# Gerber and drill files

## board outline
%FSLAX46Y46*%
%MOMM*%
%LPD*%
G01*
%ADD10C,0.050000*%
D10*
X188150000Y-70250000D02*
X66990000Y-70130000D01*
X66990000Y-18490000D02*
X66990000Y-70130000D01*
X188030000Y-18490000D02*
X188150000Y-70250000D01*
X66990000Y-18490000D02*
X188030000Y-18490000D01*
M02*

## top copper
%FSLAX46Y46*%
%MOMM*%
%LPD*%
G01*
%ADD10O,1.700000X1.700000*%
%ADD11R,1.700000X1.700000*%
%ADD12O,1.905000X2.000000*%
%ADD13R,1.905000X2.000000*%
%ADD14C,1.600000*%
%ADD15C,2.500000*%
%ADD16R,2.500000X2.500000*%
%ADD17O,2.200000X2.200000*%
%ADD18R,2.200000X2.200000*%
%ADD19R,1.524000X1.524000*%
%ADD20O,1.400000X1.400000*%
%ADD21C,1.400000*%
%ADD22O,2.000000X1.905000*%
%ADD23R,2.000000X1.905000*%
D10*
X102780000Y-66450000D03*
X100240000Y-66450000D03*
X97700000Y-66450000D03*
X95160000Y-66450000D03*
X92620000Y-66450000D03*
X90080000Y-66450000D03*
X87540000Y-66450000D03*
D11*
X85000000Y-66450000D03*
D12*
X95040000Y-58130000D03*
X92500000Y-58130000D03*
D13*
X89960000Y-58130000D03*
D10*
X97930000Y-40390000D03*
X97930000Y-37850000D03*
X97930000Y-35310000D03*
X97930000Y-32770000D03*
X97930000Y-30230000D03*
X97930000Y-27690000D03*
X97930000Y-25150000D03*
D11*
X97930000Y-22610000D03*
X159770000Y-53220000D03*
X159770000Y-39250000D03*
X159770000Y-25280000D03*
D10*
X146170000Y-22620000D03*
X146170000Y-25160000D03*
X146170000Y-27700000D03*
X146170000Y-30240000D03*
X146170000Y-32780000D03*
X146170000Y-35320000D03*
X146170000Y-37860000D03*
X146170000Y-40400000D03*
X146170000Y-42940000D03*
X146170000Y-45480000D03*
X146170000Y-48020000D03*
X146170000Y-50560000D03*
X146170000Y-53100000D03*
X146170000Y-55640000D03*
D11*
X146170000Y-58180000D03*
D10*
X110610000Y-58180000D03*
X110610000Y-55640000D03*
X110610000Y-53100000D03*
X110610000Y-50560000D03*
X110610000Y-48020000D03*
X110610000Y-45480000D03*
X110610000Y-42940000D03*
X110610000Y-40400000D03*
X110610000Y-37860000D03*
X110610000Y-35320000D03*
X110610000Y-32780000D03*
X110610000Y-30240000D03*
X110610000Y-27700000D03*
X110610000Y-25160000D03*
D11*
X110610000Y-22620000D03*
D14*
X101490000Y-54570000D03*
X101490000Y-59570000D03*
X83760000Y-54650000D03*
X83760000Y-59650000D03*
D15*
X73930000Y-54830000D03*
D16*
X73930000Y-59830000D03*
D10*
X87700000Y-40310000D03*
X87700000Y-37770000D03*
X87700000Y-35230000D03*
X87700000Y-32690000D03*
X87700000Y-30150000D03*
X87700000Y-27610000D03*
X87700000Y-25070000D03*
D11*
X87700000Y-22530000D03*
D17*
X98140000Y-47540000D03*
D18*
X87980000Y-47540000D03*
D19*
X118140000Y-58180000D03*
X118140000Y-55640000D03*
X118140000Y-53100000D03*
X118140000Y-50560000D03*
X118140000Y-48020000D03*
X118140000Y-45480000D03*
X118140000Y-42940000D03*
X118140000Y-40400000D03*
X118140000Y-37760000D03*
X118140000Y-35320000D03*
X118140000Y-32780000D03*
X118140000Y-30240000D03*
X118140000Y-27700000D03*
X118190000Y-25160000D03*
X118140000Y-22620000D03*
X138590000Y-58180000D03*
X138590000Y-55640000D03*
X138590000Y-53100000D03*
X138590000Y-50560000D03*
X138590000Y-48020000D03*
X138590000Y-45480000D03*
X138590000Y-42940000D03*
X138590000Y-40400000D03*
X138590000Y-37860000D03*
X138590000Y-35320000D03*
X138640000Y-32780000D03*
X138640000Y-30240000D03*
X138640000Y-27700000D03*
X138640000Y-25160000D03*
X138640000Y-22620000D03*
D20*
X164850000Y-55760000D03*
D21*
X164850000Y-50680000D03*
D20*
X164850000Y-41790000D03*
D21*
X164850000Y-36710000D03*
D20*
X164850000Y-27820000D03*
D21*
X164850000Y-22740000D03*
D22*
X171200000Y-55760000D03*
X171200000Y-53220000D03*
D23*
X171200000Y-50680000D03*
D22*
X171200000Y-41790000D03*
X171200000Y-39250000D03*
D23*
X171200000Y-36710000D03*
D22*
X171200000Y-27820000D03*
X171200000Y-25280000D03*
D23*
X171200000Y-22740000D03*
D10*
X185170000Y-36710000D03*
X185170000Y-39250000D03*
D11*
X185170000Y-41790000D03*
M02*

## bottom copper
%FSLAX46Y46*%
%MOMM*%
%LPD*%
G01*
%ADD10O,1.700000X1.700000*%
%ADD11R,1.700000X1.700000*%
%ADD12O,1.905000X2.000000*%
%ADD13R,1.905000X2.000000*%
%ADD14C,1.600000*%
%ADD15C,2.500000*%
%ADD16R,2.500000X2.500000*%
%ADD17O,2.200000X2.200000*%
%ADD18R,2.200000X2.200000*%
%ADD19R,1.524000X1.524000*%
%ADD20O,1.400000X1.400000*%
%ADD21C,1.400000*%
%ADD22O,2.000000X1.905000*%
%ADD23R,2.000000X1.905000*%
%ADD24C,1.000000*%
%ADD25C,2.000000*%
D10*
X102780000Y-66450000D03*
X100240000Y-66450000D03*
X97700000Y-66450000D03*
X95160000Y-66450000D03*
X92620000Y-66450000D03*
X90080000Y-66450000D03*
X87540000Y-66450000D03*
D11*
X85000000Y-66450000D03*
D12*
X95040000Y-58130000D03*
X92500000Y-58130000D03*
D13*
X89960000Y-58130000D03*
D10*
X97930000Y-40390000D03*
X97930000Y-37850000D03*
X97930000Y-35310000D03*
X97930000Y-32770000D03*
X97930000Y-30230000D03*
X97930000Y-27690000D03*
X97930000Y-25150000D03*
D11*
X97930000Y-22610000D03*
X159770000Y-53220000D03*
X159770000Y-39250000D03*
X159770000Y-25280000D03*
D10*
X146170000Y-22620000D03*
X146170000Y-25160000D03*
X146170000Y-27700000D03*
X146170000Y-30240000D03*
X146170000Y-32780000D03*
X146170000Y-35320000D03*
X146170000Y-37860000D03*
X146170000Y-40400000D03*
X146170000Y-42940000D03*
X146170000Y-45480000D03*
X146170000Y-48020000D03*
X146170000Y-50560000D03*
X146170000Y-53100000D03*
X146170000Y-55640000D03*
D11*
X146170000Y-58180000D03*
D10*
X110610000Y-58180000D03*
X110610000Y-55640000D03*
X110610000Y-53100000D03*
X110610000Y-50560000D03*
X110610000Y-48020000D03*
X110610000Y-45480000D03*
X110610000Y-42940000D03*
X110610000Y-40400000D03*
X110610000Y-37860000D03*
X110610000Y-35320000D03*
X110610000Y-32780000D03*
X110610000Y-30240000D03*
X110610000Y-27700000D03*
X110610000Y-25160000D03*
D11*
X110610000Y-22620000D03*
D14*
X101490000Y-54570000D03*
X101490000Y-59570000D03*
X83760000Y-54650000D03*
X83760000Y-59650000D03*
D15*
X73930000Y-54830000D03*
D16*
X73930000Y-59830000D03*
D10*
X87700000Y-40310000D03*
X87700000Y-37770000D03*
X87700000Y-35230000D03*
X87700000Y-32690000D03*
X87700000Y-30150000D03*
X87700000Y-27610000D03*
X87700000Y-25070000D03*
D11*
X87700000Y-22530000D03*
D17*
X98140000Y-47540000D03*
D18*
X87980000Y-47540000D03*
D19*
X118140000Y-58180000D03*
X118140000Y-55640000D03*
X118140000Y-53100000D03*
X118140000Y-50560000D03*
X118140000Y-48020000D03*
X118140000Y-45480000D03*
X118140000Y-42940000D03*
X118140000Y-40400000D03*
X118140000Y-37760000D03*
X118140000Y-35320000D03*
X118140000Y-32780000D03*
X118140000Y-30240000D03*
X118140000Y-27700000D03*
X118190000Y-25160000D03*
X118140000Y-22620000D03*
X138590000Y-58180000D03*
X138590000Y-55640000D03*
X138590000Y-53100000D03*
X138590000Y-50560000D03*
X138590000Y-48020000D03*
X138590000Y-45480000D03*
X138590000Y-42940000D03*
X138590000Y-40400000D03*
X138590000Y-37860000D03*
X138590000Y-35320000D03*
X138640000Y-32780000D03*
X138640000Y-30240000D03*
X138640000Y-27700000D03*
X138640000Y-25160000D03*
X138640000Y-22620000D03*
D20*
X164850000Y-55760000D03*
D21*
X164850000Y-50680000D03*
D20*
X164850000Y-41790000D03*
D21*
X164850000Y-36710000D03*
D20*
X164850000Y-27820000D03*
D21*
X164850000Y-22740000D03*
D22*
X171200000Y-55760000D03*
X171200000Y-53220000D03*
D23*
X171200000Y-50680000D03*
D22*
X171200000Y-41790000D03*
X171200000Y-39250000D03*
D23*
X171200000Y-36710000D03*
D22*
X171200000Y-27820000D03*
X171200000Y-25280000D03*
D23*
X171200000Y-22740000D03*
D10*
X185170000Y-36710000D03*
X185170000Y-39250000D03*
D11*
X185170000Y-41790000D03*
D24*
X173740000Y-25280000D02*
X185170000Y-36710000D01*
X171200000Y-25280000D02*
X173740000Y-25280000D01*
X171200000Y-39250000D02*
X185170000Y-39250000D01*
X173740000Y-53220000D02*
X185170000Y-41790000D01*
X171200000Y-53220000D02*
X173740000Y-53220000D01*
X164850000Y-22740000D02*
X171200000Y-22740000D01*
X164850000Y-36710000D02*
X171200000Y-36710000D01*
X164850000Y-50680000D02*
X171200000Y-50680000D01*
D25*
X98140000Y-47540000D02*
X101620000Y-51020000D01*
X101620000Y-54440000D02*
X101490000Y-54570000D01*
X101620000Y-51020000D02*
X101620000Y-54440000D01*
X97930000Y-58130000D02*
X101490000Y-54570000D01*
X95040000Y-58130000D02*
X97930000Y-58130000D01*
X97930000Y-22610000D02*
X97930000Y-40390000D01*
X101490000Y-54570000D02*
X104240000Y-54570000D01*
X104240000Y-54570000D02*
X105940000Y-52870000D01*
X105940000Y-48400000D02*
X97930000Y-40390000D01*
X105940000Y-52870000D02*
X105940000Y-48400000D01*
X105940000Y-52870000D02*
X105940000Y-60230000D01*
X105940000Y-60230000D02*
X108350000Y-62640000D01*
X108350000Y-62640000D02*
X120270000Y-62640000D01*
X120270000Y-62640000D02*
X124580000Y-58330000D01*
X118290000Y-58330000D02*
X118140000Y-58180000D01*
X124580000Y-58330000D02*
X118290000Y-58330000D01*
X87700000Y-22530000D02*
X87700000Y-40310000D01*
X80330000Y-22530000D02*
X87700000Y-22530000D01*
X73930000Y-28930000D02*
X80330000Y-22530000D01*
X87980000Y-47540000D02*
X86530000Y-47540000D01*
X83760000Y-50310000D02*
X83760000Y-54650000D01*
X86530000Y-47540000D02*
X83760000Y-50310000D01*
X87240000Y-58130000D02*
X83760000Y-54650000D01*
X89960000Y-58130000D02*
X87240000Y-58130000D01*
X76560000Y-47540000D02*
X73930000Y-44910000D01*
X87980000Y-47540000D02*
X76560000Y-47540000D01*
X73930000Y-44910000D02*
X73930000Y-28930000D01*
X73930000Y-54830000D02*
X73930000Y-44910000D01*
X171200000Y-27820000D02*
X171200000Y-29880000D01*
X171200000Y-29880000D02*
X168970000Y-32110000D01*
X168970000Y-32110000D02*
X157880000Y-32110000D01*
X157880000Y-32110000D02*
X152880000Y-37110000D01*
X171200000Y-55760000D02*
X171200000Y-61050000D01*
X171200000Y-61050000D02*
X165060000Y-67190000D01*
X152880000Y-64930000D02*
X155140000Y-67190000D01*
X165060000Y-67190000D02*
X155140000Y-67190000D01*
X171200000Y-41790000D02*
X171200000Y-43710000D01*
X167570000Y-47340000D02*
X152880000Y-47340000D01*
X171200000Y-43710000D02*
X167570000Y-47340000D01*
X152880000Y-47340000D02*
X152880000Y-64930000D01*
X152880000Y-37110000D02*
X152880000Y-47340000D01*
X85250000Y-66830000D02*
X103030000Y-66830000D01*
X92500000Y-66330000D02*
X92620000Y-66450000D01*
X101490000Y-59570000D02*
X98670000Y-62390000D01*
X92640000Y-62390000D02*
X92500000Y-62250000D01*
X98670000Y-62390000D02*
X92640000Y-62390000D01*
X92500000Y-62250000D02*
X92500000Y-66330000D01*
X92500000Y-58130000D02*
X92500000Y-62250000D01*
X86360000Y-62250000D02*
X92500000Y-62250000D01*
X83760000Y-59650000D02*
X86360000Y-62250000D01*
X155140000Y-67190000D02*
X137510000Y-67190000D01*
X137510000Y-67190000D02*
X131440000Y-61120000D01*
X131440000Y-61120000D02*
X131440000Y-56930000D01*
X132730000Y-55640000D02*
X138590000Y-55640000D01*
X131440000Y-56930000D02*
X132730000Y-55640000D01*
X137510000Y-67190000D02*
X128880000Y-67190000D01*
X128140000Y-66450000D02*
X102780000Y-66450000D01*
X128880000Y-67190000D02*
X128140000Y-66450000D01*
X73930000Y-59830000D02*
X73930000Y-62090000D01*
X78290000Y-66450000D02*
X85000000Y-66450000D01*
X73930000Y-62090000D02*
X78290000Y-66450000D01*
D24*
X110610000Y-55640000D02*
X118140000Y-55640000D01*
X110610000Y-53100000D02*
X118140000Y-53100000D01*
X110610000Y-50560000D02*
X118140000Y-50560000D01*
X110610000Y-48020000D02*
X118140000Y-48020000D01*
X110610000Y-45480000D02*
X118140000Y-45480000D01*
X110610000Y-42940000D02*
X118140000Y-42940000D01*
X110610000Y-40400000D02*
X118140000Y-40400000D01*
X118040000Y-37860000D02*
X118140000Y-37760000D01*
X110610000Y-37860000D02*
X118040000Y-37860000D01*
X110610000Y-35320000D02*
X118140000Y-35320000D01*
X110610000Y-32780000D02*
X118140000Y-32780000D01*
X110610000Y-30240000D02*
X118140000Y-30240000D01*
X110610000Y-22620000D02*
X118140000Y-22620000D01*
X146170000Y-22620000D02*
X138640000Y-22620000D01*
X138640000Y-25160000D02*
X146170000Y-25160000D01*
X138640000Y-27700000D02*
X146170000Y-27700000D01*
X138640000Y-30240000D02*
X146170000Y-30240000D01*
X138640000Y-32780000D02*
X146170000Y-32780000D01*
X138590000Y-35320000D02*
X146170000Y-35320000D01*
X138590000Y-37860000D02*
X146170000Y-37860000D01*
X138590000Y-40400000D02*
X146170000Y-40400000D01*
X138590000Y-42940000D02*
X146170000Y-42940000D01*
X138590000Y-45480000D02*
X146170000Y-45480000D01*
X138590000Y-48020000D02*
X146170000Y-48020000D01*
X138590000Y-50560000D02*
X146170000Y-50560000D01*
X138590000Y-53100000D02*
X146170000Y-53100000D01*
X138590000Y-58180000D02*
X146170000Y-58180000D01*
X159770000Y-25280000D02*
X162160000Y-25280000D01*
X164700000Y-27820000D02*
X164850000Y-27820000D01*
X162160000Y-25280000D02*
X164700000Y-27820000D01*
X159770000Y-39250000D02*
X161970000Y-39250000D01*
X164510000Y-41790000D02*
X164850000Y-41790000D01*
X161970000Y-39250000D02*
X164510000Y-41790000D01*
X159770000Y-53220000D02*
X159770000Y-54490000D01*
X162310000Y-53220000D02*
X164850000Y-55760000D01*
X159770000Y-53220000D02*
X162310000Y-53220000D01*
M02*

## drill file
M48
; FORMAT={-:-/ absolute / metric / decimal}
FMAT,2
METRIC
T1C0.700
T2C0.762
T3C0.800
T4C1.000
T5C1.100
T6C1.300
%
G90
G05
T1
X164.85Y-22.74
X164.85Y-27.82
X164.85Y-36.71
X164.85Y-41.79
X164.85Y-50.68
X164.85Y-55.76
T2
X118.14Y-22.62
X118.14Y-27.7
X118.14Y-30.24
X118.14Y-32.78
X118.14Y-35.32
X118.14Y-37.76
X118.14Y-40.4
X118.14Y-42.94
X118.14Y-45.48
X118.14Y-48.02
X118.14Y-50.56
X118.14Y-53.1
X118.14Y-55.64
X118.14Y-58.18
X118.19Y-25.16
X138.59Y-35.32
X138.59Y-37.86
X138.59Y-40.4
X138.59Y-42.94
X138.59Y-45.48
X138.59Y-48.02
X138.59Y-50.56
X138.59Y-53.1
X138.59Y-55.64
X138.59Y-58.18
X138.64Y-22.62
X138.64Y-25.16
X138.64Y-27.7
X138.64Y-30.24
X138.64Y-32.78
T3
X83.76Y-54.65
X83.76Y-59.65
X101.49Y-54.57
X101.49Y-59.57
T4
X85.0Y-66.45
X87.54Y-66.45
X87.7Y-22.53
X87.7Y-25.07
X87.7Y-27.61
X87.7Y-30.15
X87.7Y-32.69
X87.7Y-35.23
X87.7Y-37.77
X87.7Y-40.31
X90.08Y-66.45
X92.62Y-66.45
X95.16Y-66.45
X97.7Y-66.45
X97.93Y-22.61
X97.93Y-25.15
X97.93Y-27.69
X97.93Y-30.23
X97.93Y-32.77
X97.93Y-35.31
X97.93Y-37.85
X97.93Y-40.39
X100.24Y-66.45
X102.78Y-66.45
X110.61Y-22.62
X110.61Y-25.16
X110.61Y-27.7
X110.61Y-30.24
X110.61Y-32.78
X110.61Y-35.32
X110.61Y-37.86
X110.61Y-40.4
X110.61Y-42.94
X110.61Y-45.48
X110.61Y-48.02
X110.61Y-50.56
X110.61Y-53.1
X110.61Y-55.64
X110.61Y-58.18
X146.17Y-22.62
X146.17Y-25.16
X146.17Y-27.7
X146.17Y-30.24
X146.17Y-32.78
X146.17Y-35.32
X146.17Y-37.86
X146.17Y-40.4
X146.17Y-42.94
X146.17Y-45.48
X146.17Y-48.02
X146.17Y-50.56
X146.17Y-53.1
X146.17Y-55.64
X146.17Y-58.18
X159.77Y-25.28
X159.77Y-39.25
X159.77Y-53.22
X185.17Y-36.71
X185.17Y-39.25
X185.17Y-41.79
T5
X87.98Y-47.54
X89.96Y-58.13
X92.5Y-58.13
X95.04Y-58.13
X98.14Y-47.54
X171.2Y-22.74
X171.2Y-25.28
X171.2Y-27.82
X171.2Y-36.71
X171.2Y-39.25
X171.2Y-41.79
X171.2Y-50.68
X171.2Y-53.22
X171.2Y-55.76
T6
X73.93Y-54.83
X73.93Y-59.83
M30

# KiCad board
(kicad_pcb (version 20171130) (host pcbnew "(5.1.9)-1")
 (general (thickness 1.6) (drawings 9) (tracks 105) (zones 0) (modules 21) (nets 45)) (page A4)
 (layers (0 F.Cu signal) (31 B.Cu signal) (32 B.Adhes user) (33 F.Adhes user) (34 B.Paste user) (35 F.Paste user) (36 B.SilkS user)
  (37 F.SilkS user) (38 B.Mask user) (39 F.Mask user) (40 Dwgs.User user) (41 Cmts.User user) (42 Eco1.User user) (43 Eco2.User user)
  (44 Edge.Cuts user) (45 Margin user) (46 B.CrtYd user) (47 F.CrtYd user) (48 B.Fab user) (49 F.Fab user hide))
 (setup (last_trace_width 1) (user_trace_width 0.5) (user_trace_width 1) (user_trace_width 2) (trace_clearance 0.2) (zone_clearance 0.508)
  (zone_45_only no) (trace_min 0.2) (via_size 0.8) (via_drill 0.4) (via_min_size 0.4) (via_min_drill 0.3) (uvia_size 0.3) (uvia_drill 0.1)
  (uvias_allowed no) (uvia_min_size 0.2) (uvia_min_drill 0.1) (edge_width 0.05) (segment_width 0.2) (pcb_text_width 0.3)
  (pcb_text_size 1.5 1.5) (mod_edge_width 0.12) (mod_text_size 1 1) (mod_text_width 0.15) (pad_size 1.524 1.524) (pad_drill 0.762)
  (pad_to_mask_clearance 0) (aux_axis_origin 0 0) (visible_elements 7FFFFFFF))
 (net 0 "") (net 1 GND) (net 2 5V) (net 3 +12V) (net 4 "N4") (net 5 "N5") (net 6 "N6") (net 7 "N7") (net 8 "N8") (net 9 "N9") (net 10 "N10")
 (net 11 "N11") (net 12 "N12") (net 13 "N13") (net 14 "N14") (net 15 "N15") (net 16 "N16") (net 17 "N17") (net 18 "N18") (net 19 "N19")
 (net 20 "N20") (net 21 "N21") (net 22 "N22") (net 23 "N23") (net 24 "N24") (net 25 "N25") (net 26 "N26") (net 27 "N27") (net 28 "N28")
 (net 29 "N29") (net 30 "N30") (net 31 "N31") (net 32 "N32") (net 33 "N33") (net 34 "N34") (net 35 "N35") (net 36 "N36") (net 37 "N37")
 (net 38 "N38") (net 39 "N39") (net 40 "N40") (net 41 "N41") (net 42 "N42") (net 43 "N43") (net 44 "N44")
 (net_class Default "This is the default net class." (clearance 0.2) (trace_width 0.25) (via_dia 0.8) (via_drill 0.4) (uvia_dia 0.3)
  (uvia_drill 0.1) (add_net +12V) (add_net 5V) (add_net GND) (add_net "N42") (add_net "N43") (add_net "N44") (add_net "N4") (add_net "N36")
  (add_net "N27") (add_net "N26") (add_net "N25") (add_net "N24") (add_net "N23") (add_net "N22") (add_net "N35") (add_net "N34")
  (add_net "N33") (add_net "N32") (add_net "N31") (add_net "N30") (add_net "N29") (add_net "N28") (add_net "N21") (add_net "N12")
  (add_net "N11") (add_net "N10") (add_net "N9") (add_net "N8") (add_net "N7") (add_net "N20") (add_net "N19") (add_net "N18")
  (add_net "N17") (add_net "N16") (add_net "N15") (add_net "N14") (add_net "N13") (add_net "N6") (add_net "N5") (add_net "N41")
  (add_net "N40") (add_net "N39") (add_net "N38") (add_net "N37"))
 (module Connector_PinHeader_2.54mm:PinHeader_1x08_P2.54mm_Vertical (layer F.Cu) (at 85 66.45 90)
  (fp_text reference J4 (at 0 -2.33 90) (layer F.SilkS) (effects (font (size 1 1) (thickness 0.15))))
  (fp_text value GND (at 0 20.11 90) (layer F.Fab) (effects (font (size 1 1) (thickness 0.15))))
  (pad 8 thru_hole oval (at 0 17.78 90) (size 1.7 1.7) (drill 1) (layers *.Cu *.Mask) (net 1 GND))
  (pad 7 thru_hole oval (at 0 15.24 90) (size 1.7 1.7) (drill 1) (layers *.Cu *.Mask) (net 1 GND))
  (pad 6 thru_hole oval (at 0 12.7 90) (size 1.7 1.7) (drill 1) (layers *.Cu *.Mask) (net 1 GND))
  (pad 5 thru_hole oval (at 0 10.16 90) (size 1.7 1.7) (drill 1) (layers *.Cu *.Mask) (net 1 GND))
  (pad 4 thru_hole oval (at 0 7.62 90) (size 1.7 1.7) (drill 1) (layers *.Cu *.Mask) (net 1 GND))
  (pad 3 thru_hole oval (at 0 5.08 90) (size 1.7 1.7) (drill 1) (layers *.Cu *.Mask) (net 1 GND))
  (pad 2 thru_hole oval (at 0 2.54 90) (size 1.7 1.7) (drill 1) (layers *.Cu *.Mask) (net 1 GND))
  (pad 1 thru_hole rect (at 0 0 90) (size 1.7 1.7) (drill 1) (layers *.Cu *.Mask) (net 1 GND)))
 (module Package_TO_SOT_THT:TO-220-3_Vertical (layer F.Cu) (at 89.96 58.13)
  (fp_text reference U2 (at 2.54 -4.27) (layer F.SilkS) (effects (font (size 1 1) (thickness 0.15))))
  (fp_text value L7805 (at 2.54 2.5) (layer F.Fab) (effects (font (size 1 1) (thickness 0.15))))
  (pad 3 thru_hole oval (at 5.08 0) (size 1.905 2) (drill 1.1) (layers *.Cu *.Mask) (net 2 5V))
  (pad 2 thru_hole oval (at 2.54 0) (size 1.905 2) (drill 1.1) (layers *.Cu *.Mask) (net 1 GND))
  (pad 1 thru_hole rect (at 0 0) (size 1.905 2) (drill 1.1) (layers *.Cu *.Mask) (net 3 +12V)))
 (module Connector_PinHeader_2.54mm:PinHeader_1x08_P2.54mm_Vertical (layer F.Cu) (at 97.93 22.61)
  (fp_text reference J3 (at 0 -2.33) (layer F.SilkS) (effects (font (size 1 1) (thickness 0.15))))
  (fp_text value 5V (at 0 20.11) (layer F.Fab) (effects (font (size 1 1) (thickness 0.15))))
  (pad 8 thru_hole oval (at 0 17.78) (size 1.7 1.7) (drill 1) (layers *.Cu *.Mask) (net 2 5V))
  (pad 7 thru_hole oval (at 0 15.24) (size 1.7 1.7) (drill 1) (layers *.Cu *.Mask) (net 2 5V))
  (pad 6 thru_hole oval (at 0 12.7) (size 1.7 1.7) (drill 1) (layers *.Cu *.Mask) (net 2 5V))
  (pad 5 thru_hole oval (at 0 10.16) (size 1.7 1.7) (drill 1) (layers *.Cu *.Mask) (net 2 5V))
  (pad 4 thru_hole oval (at 0 7.62) (size 1.7 1.7) (drill 1) (layers *.Cu *.Mask) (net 2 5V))
  (pad 3 thru_hole oval (at 0 5.08) (size 1.7 1.7) (drill 1) (layers *.Cu *.Mask) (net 2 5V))
  (pad 2 thru_hole oval (at 0 2.54) (size 1.7 1.7) (drill 1) (layers *.Cu *.Mask) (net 2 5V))
  (pad 1 thru_hole rect (at 0 0) (size 1.7 1.7) (drill 1) (layers *.Cu *.Mask) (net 2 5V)))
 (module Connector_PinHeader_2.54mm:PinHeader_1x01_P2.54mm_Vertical (layer F.Cu) (at 159.77 53.22)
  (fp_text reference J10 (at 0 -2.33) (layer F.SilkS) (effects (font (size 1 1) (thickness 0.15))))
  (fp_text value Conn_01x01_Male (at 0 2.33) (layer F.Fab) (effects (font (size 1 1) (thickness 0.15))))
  (pad 1 thru_hole rect (at 0 0) (size 1.7 1.7) (drill 1) (layers *.Cu *.Mask) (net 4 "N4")))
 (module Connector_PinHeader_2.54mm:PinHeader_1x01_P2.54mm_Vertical (layer F.Cu) (at 159.77 39.25)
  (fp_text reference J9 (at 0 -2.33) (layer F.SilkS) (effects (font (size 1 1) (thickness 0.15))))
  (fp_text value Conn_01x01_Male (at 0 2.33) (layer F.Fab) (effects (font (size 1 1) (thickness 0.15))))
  (pad 1 thru_hole rect (at 0 0) (size 1.7 1.7) (drill 1) (layers *.Cu *.Mask) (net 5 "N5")))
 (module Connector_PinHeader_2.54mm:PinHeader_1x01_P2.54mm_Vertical (layer F.Cu) (at 159.77 25.28)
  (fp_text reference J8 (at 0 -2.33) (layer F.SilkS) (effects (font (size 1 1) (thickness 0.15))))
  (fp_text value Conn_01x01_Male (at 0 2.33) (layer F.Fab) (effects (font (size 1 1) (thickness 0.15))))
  (pad 1 thru_hole rect (at 0 0) (size 1.7 1.7) (drill 1) (layers *.Cu *.Mask) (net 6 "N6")))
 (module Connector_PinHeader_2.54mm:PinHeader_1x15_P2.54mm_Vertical (layer F.Cu) (at 146.17 58.18 180)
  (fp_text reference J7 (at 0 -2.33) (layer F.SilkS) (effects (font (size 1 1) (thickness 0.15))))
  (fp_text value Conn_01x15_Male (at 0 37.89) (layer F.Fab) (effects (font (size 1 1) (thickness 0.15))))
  (pad 15 thru_hole oval (at 0 35.56 180) (size 1.7 1.7) (drill 1) (layers *.Cu *.Mask) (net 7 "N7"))
  (pad 14 thru_hole oval (at 0 33.02 180) (size 1.7 1.7) (drill 1) (layers *.Cu *.Mask) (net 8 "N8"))
  (pad 13 thru_hole oval (at 0 30.48 180) (size 1.7 1.7) (drill 1) (layers *.Cu *.Mask) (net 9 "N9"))
  (pad 12 thru_hole oval (at 0 27.94 180) (size 1.7 1.7) (drill 1) (layers *.Cu *.Mask) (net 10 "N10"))
  (pad 11 thru_hole oval (at 0 25.4 180) (size 1.7 1.7) (drill 1) (layers *.Cu *.Mask) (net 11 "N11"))
  (pad 10 thru_hole oval (at 0 22.86 180) (size 1.7 1.7) (drill 1) (layers *.Cu *.Mask) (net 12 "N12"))
  (pad 9 thru_hole oval (at 0 20.32 180) (size 1.7 1.7) (drill 1) (layers *.Cu *.Mask) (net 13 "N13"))
  (pad 8 thru_hole oval (at 0 17.78 180) (size 1.7 1.7) (drill 1) (layers *.Cu *.Mask) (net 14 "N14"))
  (pad 7 thru_hole oval (at 0 15.24 180) (size 1.7 1.7) (drill 1) (layers *.Cu *.Mask) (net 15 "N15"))
  (pad 6 thru_hole oval (at 0 12.7 180) (size 1.7 1.7) (drill 1) (layers *.Cu *.Mask) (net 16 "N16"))
  (pad 5 thru_hole oval (at 0 10.16 180) (size 1.7 1.7) (drill 1) (layers *.Cu *.Mask) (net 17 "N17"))
  (pad 4 thru_hole oval (at 0 7.62 180) (size 1.7 1.7) (drill 1) (layers *.Cu *.Mask) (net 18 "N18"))
  (pad 3 thru_hole oval (at 0 5.08 180) (size 1.7 1.7) (drill 1) (layers *.Cu *.Mask) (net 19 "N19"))
  (pad 2 thru_hole oval (at 0 2.54 180) (size 1.7 1.7) (drill 1) (layers *.Cu *.Mask) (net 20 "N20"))
  (pad 1 thru_hole rect (at 0 0 180) (size 1.7 1.7) (drill 1) (layers *.Cu *.Mask) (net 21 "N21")))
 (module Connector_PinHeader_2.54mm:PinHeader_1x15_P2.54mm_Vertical (layer F.Cu) (at 110.61 22.62)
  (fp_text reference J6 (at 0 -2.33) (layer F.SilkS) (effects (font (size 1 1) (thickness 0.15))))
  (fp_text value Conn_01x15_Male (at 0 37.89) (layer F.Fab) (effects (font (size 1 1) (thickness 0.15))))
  (pad 15 thru_hole oval (at 0 35.56) (size 1.7 1.7) (drill 1) (layers *.Cu *.Mask) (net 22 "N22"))
  (pad 14 thru_hole oval (at 0 33.02) (size 1.7 1.7) (drill 1) (layers *.Cu *.Mask) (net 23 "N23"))
  (pad 13 thru_hole oval (at 0 30.48) (size 1.7 1.7) (drill 1) (layers *.Cu *.Mask) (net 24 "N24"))
  (pad 12 thru_hole oval (at 0 27.94) (size 1.7 1.7) (drill 1) (layers *.Cu *.Mask) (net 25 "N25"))
  (pad 11 thru_hole oval (at 0 25.4) (size 1.7 1.7) (drill 1) (layers *.Cu *.Mask) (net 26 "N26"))
  (pad 10 thru_hole oval (at 0 22.86) (size 1.7 1.7) (drill 1) (layers *.Cu *.Mask) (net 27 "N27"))
  (pad 9 thru_hole oval (at 0 20.32) (size 1.7 1.7) (drill 1) (layers *.Cu *.Mask) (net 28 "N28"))
  (pad 8 thru_hole oval (at 0 17.78) (size 1.7 1.7) (drill 1) (layers *.Cu *.Mask) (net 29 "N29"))
  (pad 7 thru_hole oval (at 0 15.24) (size 1.7 1.7) (drill 1) (layers *.Cu *.Mask) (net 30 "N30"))
  (pad 6 thru_hole oval (at 0 12.7) (size 1.7 1.7) (drill 1) (layers *.Cu *.Mask) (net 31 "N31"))
  (pad 5 thru_hole oval (at 0 10.16) (size 1.7 1.7) (drill 1) (layers *.Cu *.Mask) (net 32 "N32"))
  (pad 4 thru_hole oval (at 0 7.62) (size 1.7 1.7) (drill 1) (layers *.Cu *.Mask) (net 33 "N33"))
  (pad 3 thru_hole oval (at 0 5.08) (size 1.7 1.7) (drill 1) (layers *.Cu *.Mask) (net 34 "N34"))
  (pad 2 thru_hole oval (at 0 2.54) (size 1.7 1.7) (drill 1) (layers *.Cu *.Mask) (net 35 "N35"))
  (pad 1 thru_hole rect (at 0 0) (size 1.7 1.7) (drill 1) (layers *.Cu *.Mask) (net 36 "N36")))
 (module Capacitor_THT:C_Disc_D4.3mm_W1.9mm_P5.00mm (layer F.Cu) (at 101.49 59.57 90)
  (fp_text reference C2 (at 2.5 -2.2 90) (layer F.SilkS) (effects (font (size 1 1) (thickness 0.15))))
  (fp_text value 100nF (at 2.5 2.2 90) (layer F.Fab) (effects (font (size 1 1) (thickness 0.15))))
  (pad 2 thru_hole circle (at 5 0 90) (size 1.6 1.6) (drill 0.8) (layers *.Cu *.Mask) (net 2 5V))
  (pad 1 thru_hole circle (at 0 0 90) (size 1.6 1.6) (drill 0.8) (layers *.Cu *.Mask) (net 1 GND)))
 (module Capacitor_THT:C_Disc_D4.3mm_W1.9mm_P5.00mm (layer F.Cu) (at 83.76 59.65 90)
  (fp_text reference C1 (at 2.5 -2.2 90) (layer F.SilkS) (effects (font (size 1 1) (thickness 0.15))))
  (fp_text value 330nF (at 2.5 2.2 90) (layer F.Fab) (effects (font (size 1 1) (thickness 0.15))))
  (pad 2 thru_hole circle (at 5 0 90) (size 1.6 1.6) (drill 0.8) (layers *.Cu *.Mask) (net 3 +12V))
  (pad 1 thru_hole circle (at 0 0 90) (size 1.6 1.6) (drill 0.8) (layers *.Cu *.Mask) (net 1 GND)))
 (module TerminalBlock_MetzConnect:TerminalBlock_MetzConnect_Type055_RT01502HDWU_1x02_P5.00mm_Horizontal (layer F.Cu) (at 73.93 59.83 90)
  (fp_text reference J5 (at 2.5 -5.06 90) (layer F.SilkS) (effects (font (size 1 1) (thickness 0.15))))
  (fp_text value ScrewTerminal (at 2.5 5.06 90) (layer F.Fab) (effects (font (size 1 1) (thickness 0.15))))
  (pad 2 thru_hole circle (at 5 0 90) (size 2.5 2.5) (drill 1.3) (layers *.Cu *.Mask) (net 3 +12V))
  (pad 1 thru_hole rect (at 0 0 90) (size 2.5 2.5) (drill 1.3) (layers *.Cu *.Mask) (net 1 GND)))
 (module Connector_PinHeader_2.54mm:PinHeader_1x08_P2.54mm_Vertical (layer F.Cu) (at 87.7 22.53)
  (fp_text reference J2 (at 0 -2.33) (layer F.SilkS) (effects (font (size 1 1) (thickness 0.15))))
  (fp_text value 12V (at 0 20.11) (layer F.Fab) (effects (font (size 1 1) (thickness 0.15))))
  (pad 8 thru_hole oval (at 0 17.78) (size 1.7 1.7) (drill 1) (layers *.Cu *.Mask) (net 3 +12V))
  (pad 7 thru_hole oval (at 0 15.24) (size 1.7 1.7) (drill 1) (layers *.Cu *.Mask) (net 3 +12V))
  (pad 6 thru_hole oval (at 0 12.7) (size 1.7 1.7) (drill 1) (layers *.Cu *.Mask) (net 3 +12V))
  (pad 5 thru_hole oval (at 0 10.16) (size 1.7 1.7) (drill 1) (layers *.Cu *.Mask) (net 3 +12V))
  (pad 4 thru_hole oval (at 0 7.62) (size 1.7 1.7) (drill 1) (layers *.Cu *.Mask) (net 3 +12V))
  (pad 3 thru_hole oval (at 0 5.08) (size 1.7 1.7) (drill 1) (layers *.Cu *.Mask) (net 3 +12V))
  (pad 2 thru_hole oval (at 0 2.54) (size 1.7 1.7) (drill 1) (layers *.Cu *.Mask) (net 3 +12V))
  (pad 1 thru_hole rect (at 0 0) (size 1.7 1.7) (drill 1) (layers *.Cu *.Mask) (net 3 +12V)))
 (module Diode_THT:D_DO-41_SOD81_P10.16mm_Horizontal (layer F.Cu) (at 87.98 47.54)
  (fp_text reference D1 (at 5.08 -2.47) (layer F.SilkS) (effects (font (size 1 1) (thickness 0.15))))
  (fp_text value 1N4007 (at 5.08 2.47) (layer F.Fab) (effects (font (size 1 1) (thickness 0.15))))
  (pad 2 thru_hole oval (at 10.16 0) (size 2.2 2.2) (drill 1.1) (layers *.Cu *.Mask) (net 2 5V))
  (pad 1 thru_hole rect (at 0 0) (size 2.2 2.2) (drill 1.1) (layers *.Cu *.Mask) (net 3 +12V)))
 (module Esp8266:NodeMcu (layer F.Cu) (at 128.39 37.86)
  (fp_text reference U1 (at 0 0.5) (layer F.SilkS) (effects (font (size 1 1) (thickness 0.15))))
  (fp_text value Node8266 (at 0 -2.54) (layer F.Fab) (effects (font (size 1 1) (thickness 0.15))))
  (pad 30 thru_hole rect (at -10.25 20.32) (size 1.524 1.524) (drill 0.762) (layers *.Cu *.Mask) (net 2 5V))
  (pad 29 thru_hole rect (at -10.25 17.78) (size 1.524 1.524) (drill 0.762) (layers *.Cu *.Mask) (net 23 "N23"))
  (pad 28 thru_hole rect (at -10.25 15.24) (size 1.524 1.524) (drill 0.762) (layers *.Cu *.Mask) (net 24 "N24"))
  (pad 27 thru_hole rect (at -10.25 12.7) (size 1.524 1.524) (drill 0.762) (layers *.Cu *.Mask) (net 25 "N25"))
  (pad 26 thru_hole rect (at -10.25 10.16) (size 1.524 1.524) (drill 0.762) (layers *.Cu *.Mask) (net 26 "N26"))
  (pad 25 thru_hole rect (at -10.25 7.62) (size 1.524 1.524) (drill 0.762) (layers *.Cu *.Mask) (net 27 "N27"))
  (pad 24 thru_hole rect (at -10.25 5.08) (size 1.524 1.524) (drill 0.762) (layers *.Cu *.Mask) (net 28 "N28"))
  (pad 23 thru_hole rect (at -10.25 2.54) (size 1.524 1.524) (drill 0.762) (layers *.Cu *.Mask) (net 29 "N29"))
  (pad 22 thru_hole rect (at -10.25 -0.1) (size 1.524 1.524) (drill 0.762) (layers *.Cu *.Mask) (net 30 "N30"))
  (pad 21 thru_hole rect (at -10.25 -2.54) (size 1.524 1.524) (drill 0.762) (layers *.Cu *.Mask) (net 31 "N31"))
  (pad 20 thru_hole rect (at -10.25 -5.08) (size 1.524 1.524) (drill 0.762) (layers *.Cu *.Mask) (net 32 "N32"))
  (pad 19 thru_hole rect (at -10.25 -7.62) (size 1.524 1.524) (drill 0.762) (layers *.Cu *.Mask) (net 33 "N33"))
  (pad 18 thru_hole rect (at -10.25 -10.16) (size 1.524 1.524) (drill 0.762) (layers *.Cu *.Mask) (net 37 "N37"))
  (pad 17 thru_hole rect (at -10.2 -12.7) (size 1.524 1.524) (drill 0.762) (layers *.Cu *.Mask) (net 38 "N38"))
  (pad 16 thru_hole rect (at -10.25 -15.24) (size 1.524 1.524) (drill 0.762) (layers *.Cu *.Mask) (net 36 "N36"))
  (pad 15 thru_hole rect (at 10.2 20.32) (size 1.524 1.524) (drill 0.762) (layers *.Cu *.Mask) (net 21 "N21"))
  (pad 14 thru_hole rect (at 10.2 17.78) (size 1.524 1.524) (drill 0.762) (layers *.Cu *.Mask) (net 1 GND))
  (pad 13 thru_hole rect (at 10.2 15.24) (size 1.524 1.524) (drill 0.762) (layers *.Cu *.Mask) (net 19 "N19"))
  (pad 12 thru_hole rect (at 10.2 12.7) (size 1.524 1.524) (drill 0.762) (layers *.Cu *.Mask) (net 18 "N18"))
  (pad 11 thru_hole rect (at 10.2 10.16) (size 1.524 1.524) (drill 0.762) (layers *.Cu *.Mask) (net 17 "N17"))
  (pad 10 thru_hole rect (at 10.2 7.62) (size 1.524 1.524) (drill 0.762) (layers *.Cu *.Mask) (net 16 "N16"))
  (pad 9 thru_hole rect (at 10.2 5.08 90) (size 1.524 1.524) (drill 0.762) (layers *.Cu *.Mask) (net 15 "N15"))
  (pad 8 thru_hole rect (at 10.2 2.54) (size 1.524 1.524) (drill 0.762) (layers *.Cu *.Mask) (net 14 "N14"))
  (pad 7 thru_hole rect (at 10.2 0) (size 1.524 1.524) (drill 0.762) (layers *.Cu *.Mask) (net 13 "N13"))
  (pad 6 thru_hole rect (at 10.2 -2.54) (size 1.524 1.524) (drill 0.762) (layers *.Cu *.Mask) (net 12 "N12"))
  (pad 5 thru_hole rect (at 10.25 -5.08) (size 1.524 1.524) (drill 0.762) (layers *.Cu *.Mask) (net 11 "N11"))
  (pad 4 thru_hole rect (at 10.25 -7.62) (size 1.524 1.524) (drill 0.762) (layers *.Cu *.Mask) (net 10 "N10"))
  (pad 3 thru_hole rect (at 10.25 -10.16) (size 1.524 1.524) (drill 0.762) (layers *.Cu *.Mask) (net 9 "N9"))
  (pad 2 thru_hole rect (at 10.25 -12.7) (size 1.524 1.524) (drill 0.762) (layers *.Cu *.Mask) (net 8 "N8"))
  (pad 1 thru_hole rect (at 10.25 -15.24) (size 1.524 1.524) (drill 0.762) (layers *.Cu *.Mask) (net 7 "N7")))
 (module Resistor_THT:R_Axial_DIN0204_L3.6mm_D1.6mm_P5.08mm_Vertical (layer F.Cu) (at 164.85 50.68 270)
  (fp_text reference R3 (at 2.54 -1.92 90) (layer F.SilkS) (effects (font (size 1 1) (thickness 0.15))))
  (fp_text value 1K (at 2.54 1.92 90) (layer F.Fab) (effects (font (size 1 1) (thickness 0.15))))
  (pad 2 thru_hole oval (at 5.08 0 270) (size 1.4 1.4) (drill 0.7) (layers *.Cu *.Mask) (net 4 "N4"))
  (pad 1 thru_hole circle (at 0 0 270) (size 1.4 1.4) (drill 0.7) (layers *.Cu *.Mask) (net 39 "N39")))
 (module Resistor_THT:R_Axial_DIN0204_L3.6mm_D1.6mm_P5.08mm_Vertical (layer F.Cu) (at 164.85 36.71 270)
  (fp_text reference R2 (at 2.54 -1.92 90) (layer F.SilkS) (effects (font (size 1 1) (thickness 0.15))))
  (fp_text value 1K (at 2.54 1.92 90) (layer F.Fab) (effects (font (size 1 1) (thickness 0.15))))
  (pad 2 thru_hole oval (at 5.08 0 270) (size 1.4 1.4) (drill 0.7) (layers *.Cu *.Mask) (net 5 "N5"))
  (pad 1 thru_hole circle (at 0 0 270) (size 1.4 1.4) (drill 0.7) (layers *.Cu *.Mask) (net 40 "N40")))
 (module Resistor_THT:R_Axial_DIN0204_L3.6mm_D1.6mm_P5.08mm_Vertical (layer F.Cu) (at 164.85 22.74 270)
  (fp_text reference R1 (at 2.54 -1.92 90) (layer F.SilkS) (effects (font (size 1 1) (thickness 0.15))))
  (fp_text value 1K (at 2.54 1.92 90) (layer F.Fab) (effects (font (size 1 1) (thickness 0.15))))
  (pad 2 thru_hole oval (at 5.08 0 270) (size 1.4 1.4) (drill 0.7) (layers *.Cu *.Mask) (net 6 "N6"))
  (pad 1 thru_hole circle (at 0 0 270) (size 1.4 1.4) (drill 0.7) (layers *.Cu *.Mask) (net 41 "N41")))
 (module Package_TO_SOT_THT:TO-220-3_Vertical (layer F.Cu) (at 171.2 50.68 270)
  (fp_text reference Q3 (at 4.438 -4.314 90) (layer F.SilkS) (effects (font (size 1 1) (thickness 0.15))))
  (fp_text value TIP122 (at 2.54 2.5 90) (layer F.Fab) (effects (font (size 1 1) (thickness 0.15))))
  (pad 3 thru_hole oval (at 5.08 0 270) (size 1.905 2) (drill 1.1) (layers *.Cu *.Mask) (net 1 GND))
  (pad 2 thru_hole oval (at 2.54 0 270) (size 1.905 2) (drill 1.1) (layers *.Cu *.Mask) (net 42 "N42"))
  (pad 1 thru_hole rect (at 0 0 270) (size 1.905 2) (drill 1.1) (layers *.Cu *.Mask) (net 39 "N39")))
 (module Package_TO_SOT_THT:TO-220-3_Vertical (layer F.Cu) (at 171.2 36.71 270)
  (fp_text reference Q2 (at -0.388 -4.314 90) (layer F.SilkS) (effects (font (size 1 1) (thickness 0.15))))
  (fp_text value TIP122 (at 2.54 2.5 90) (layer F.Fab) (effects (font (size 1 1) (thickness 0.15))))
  (pad 3 thru_hole oval (at 5.08 0 270) (size 1.905 2) (drill 1.1) (layers *.Cu *.Mask) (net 1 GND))
  (pad 2 thru_hole oval (at 2.54 0 270) (size 1.905 2) (drill 1.1) (layers *.Cu *.Mask) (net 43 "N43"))
  (pad 1 thru_hole rect (at 0 0 270) (size 1.905 2) (drill 1.1) (layers *.Cu *.Mask) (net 40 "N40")))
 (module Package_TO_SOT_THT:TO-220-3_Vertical (layer F.Cu) (at 171.2 22.74 270)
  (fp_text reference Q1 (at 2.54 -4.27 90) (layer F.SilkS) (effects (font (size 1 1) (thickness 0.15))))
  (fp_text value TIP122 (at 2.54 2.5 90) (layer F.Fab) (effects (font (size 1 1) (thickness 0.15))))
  (pad 3 thru_hole oval (at 5.08 0 270) (size 1.905 2) (drill 1.1) (layers *.Cu *.Mask) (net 1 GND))
  (pad 2 thru_hole oval (at 2.54 0 270) (size 1.905 2) (drill 1.1) (layers *.Cu *.Mask) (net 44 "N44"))
  (pad 1 thru_hole rect (at 0 0 270) (size 1.905 2) (drill 1.1) (layers *.Cu *.Mask) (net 41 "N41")))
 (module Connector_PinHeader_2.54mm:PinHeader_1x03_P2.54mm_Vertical (layer F.Cu) (at 185.17 41.79 180)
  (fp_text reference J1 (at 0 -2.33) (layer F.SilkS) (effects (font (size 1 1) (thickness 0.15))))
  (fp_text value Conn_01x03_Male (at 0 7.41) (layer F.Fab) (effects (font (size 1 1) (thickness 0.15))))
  (pad 3 thru_hole oval (at 0 5.08 180) (size 1.7 1.7) (drill 1) (layers *.Cu *.Mask) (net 44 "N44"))
  (pad 2 thru_hole oval (at 0 2.54 180) (size 1.7 1.7) (drill 1) (layers *.Cu *.Mask) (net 43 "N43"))
  (pad 1 thru_hole rect (at 0 0 180) (size 1.7 1.7) (drill 1) (layers *.Cu *.Mask) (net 42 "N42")))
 (gr_line (start 188.15 70.25) (end 66.99 70.13) (layer Edge.Cuts) (width 0.05))
 (gr_line (start 66.99 18.49) (end 66.99 70.13) (layer Edge.Cuts) (width 0.05))
 (gr_line (start 188.03 18.49) (end 188.15 70.25) (layer Edge.Cuts) (width 0.05))
 (gr_line (start 66.99 18.49) (end 188.03 18.49) (layer Edge.Cuts) (width 0.05))
 (segment (start 173.74 25.28) (end 185.17 36.71) (width 1) (layer B.Cu) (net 44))
 (segment (start 171.2 25.28) (end 173.74 25.28) (width 1) (layer B.Cu) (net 44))
 (segment (start 171.2 39.25) (end 185.17 39.25) (width 1) (layer B.Cu) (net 43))
 (segment (start 173.74 53.22) (end 185.17 41.79) (width 1) (layer B.Cu) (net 42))
 (segment (start 171.2 53.22) (end 173.74 53.22) (width 1) (layer B.Cu) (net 42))
 (segment (start 164.85 22.74) (end 171.2 22.74) (width 1) (layer B.Cu) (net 41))
 (segment (start 164.85 36.71) (end 171.2 36.71) (width 1) (layer B.Cu) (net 40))
 (segment (start 164.85 50.68) (end 171.2 50.68) (width 1) (layer B.Cu) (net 39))
 (segment (start 98.14 47.54) (end 101.62 51.02) (width 2) (layer B.Cu) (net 2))
 (segment (start 101.62 54.44) (end 101.49 54.57) (width 2) (layer B.Cu) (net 2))
 (segment (start 101.62 51.02) (end 101.62 54.44) (width 2) (layer B.Cu) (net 2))
 (segment (start 97.93 58.13) (end 101.49 54.57) (width 2) (layer B.Cu) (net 2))
 (segment (start 95.04 58.13) (end 97.93 58.13) (width 2) (layer B.Cu) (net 2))
 (segment (start 97.93 22.61) (end 97.93 40.39) (width 2) (layer B.Cu) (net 2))
 (segment (start 101.49 54.57) (end 104.24 54.57) (width 2) (layer B.Cu) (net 2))
 (segment (start 104.24 54.57) (end 105.94 52.87) (width 2) (layer B.Cu) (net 2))
 (segment (start 105.94 48.4) (end 97.93 40.39) (width 2) (layer B.Cu) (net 2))
 (segment (start 105.94 52.87) (end 105.94 48.4) (width 2) (layer B.Cu) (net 2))
 (segment (start 105.94 52.87) (end 105.94 60.23) (width 2) (layer B.Cu) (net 2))
 (segment (start 105.94 60.23) (end 108.35 62.64) (width 2) (layer B.Cu) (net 2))
 (segment (start 108.35 62.64) (end 120.27 62.64) (width 2) (layer B.Cu) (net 2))
 (segment (start 120.27 62.64) (end 124.58 58.33) (width 2) (layer B.Cu) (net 2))
 (segment (start 118.29 58.33) (end 118.14 58.18) (width 2) (layer B.Cu) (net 2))
 (segment (start 124.58 58.33) (end 118.29 58.33) (width 2) (layer B.Cu) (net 2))
 (segment (start 87.7 22.53) (end 87.7 40.31) (width 2) (layer B.Cu) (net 3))
 (segment (start 80.33 22.53) (end 87.7 22.53) (width 2) (layer B.Cu) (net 3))
 (segment (start 73.93 28.93) (end 80.33 22.53) (width 2) (layer B.Cu) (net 3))
 (segment (start 87.98 47.54) (end 86.53 47.54) (width 2) (layer B.Cu) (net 3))
 (segment (start 83.76 50.31) (end 83.76 54.65) (width 2) (layer B.Cu) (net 3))
 (segment (start 86.53 47.54) (end 83.76 50.31) (width 2) (layer B.Cu) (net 3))
 (segment (start 87.24 58.13) (end 83.76 54.65) (width 2) (layer B.Cu) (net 3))
 (segment (start 89.96 58.13) (end 87.24 58.13) (width 2) (layer B.Cu) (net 3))
 (segment (start 76.56 47.54) (end 73.93 44.91) (width 2) (layer B.Cu) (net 3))
 (segment (start 87.98 47.54) (end 76.56 47.54) (width 2) (layer B.Cu) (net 3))
 (segment (start 73.93 44.91) (end 73.93 28.93) (width 2) (layer B.Cu) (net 3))
 (segment (start 73.93 54.83) (end 73.93 44.91) (width 2) (layer B.Cu) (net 3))
 (segment (start 171.2 27.82) (end 171.2 29.88) (width 2) (layer B.Cu) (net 1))
 (segment (start 171.2 29.88) (end 168.97 32.11) (width 2) (layer B.Cu) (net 1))
 (segment (start 168.97 32.11) (end 157.88 32.11) (width 2) (layer B.Cu) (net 1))
 (segment (start 157.88 32.11) (end 152.88 37.11) (width 2) (layer B.Cu) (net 1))
 (segment (start 171.2 55.76) (end 171.2 61.05) (width 2) (layer B.Cu) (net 1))
 (segment (start 171.2 61.05) (end 165.06 67.19) (width 2) (layer B.Cu) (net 1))
 (segment (start 152.88 64.93) (end 155.14 67.19) (width 2) (layer B.Cu) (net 1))
 (segment (start 165.06 67.19) (end 155.14 67.19) (width 2) (layer B.Cu) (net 1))
 (segment (start 171.2 41.79) (end 171.2 43.71) (width 2) (layer B.Cu) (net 1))
 (segment (start 167.57 47.34) (end 152.88 47.34) (width 2) (layer B.Cu) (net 1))
 (segment (start 171.2 43.71) (end 167.57 47.34) (width 2) (layer B.Cu) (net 1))
 (segment (start 152.88 47.34) (end 152.88 64.93) (width 2) (layer B.Cu) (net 1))
 (segment (start 152.88 37.11) (end 152.88 47.34) (width 2) (layer B.Cu) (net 1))
 (segment (start 85.25 66.83) (end 103.03 66.83) (width 2) (layer B.Cu) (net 1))
 (segment (start 92.5 66.33) (end 92.62 66.45) (width 2) (layer B.Cu) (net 1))
 (segment (start 101.49 59.57) (end 98.67 62.39) (width 2) (layer B.Cu) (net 1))
 (segment (start 92.64 62.39) (end 92.5 62.25) (width 2) (layer B.Cu) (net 1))
 (segment (start 98.67 62.39) (end 92.64 62.39) (width 2) (layer B.Cu) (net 1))
 (segment (start 92.5 62.25) (end 92.5 66.33) (width 2) (layer B.Cu) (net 1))
 (segment (start 92.5 58.13) (end 92.5 62.25) (width 2) (layer B.Cu) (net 1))
 (segment (start 86.36 62.25) (end 92.5 62.25) (width 2) (layer B.Cu) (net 1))
 (segment (start 83.76 59.65) (end 86.36 62.25) (width 2) (layer B.Cu) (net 1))
 (segment (start 155.14 67.19) (end 137.51 67.19) (width 2) (layer B.Cu) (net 1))
 (segment (start 137.51 67.19) (end 131.44 61.12) (width 2) (layer B.Cu) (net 1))
 (segment (start 131.44 61.12) (end 131.44 56.93) (width 2) (layer B.Cu) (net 1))
 (segment (start 132.73 55.64) (end 138.59 55.64) (width 2) (layer B.Cu) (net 1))
 (segment (start 131.44 56.93) (end 132.73 55.64) (width 2) (layer B.Cu) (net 1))
 (segment (start 137.51 67.19) (end 128.88 67.19) (width 2) (layer B.Cu) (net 1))
 (segment (start 128.14 66.45) (end 102.78 66.45) (width 2) (layer B.Cu) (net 1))
 (segment (start 128.88 67.19) (end 128.14 66.45) (width 2) (layer B.Cu) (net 1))
 (segment (start 73.93 59.83) (end 73.93 62.09) (width 2) (layer B.Cu) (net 1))
 (segment (start 78.29 66.45) (end 85 66.45) (width 2) (layer B.Cu) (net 1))
 (segment (start 73.93 62.09) (end 78.29 66.45) (width 2) (layer B.Cu) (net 1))
 (segment (start 110.61 55.64) (end 118.14 55.64) (width 1) (layer B.Cu) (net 23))
 (segment (start 110.61 53.1) (end 118.14 53.1) (width 1) (layer B.Cu) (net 24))
 (segment (start 110.61 50.56) (end 118.14 50.56) (width 1) (layer B.Cu) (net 25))
 (segment (start 110.61 48.02) (end 118.14 48.02) (width 1) (layer B.Cu) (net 26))
 (segment (start 110.61 45.48) (end 118.14 45.48) (width 1) (layer B.Cu) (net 27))
 (segment (start 110.61 42.94) (end 118.14 42.94) (width 1) (layer B.Cu) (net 28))
 (segment (start 110.61 40.4) (end 118.14 40.4) (width 1) (layer B.Cu) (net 29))
 (segment (start 118.04 37.86) (end 118.14 37.76) (width 1) (layer B.Cu) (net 30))
 (segment (start 110.61 37.86) (end 118.04 37.86) (width 1) (layer B.Cu) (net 30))
 (segment (start 110.61 35.32) (end 118.14 35.32) (width 1) (layer B.Cu) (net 31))
 (segment (start 110.61 32.78) (end 118.14 32.78) (width 1) (layer B.Cu) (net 32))
 (segment (start 110.61 30.24) (end 118.14 30.24) (width 1) (layer B.Cu) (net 33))
 (segment (start 110.61 22.62) (end 118.14 22.62) (width 1) (layer B.Cu) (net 36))
 (segment (start 146.17 22.62) (end 138.64 22.62) (width 1) (layer B.Cu) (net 7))
 (segment (start 138.64 25.16) (end 146.17 25.16) (width 1) (layer B.Cu) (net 8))
 (segment (start 138.64 27.7) (end 146.17 27.7) (width 1) (layer B.Cu) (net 9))
 (segment (start 138.64 30.24) (end 146.17 30.24) (width 1) (layer B.Cu) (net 10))
 (segment (start 138.64 32.78) (end 146.17 32.78) (width 1) (layer B.Cu) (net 11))
 (segment (start 138.59 35.32) (end 146.17 35.32) (width 1) (layer B.Cu) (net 12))
 (segment (start 138.59 37.86) (end 146.17 37.86) (width 1) (layer B.Cu) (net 13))
 (segment (start 138.59 40.4) (end 146.17 40.4) (width 1) (layer B.Cu) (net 14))
 (segment (start 138.59 42.94) (end 146.17 42.94) (width 1) (layer B.Cu) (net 15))
 (segment (start 138.59 45.48) (end 146.17 45.48) (width 1) (layer B.Cu) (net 16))
 (segment (start 138.59 48.02) (end 146.17 48.02) (width 1) (layer B.Cu) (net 17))
 (segment (start 138.59 50.56) (end 146.17 50.56) (width 1) (layer B.Cu) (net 18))
 (segment (start 138.59 53.1) (end 146.17 53.1) (width 1) (layer B.Cu) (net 19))
 (segment (start 138.59 58.18) (end 146.17 58.18) (width 1) (layer B.Cu) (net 21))
 (segment (start 159.77 25.28) (end 162.16 25.28) (width 1) (layer B.Cu) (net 6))
 (segment (start 164.7 27.82) (end 164.85 27.82) (width 1) (layer B.Cu) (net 6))
 (segment (start 162.16 25.28) (end 164.7 27.82) (width 1) (layer B.Cu) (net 6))
 (segment (start 159.77 39.25) (end 161.97 39.25) (width 1) (layer B.Cu) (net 5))
 (segment (start 164.51 41.79) (end 164.85 41.79) (width 1) (layer B.Cu) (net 5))
 (segment (start 161.97 39.25) (end 164.51 41.79) (width 1) (layer B.Cu) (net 5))
 (segment (start 159.77 53.22) (end 159.77 54.49) (width 1) (layer B.Cu) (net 4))
 (segment (start 162.31 53.22) (end 164.85 55.76) (width 1) (layer B.Cu) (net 4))
 (segment (start 159.77 53.22) (end 162.31 53.22) (width 1) (layer B.Cu) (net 4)))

